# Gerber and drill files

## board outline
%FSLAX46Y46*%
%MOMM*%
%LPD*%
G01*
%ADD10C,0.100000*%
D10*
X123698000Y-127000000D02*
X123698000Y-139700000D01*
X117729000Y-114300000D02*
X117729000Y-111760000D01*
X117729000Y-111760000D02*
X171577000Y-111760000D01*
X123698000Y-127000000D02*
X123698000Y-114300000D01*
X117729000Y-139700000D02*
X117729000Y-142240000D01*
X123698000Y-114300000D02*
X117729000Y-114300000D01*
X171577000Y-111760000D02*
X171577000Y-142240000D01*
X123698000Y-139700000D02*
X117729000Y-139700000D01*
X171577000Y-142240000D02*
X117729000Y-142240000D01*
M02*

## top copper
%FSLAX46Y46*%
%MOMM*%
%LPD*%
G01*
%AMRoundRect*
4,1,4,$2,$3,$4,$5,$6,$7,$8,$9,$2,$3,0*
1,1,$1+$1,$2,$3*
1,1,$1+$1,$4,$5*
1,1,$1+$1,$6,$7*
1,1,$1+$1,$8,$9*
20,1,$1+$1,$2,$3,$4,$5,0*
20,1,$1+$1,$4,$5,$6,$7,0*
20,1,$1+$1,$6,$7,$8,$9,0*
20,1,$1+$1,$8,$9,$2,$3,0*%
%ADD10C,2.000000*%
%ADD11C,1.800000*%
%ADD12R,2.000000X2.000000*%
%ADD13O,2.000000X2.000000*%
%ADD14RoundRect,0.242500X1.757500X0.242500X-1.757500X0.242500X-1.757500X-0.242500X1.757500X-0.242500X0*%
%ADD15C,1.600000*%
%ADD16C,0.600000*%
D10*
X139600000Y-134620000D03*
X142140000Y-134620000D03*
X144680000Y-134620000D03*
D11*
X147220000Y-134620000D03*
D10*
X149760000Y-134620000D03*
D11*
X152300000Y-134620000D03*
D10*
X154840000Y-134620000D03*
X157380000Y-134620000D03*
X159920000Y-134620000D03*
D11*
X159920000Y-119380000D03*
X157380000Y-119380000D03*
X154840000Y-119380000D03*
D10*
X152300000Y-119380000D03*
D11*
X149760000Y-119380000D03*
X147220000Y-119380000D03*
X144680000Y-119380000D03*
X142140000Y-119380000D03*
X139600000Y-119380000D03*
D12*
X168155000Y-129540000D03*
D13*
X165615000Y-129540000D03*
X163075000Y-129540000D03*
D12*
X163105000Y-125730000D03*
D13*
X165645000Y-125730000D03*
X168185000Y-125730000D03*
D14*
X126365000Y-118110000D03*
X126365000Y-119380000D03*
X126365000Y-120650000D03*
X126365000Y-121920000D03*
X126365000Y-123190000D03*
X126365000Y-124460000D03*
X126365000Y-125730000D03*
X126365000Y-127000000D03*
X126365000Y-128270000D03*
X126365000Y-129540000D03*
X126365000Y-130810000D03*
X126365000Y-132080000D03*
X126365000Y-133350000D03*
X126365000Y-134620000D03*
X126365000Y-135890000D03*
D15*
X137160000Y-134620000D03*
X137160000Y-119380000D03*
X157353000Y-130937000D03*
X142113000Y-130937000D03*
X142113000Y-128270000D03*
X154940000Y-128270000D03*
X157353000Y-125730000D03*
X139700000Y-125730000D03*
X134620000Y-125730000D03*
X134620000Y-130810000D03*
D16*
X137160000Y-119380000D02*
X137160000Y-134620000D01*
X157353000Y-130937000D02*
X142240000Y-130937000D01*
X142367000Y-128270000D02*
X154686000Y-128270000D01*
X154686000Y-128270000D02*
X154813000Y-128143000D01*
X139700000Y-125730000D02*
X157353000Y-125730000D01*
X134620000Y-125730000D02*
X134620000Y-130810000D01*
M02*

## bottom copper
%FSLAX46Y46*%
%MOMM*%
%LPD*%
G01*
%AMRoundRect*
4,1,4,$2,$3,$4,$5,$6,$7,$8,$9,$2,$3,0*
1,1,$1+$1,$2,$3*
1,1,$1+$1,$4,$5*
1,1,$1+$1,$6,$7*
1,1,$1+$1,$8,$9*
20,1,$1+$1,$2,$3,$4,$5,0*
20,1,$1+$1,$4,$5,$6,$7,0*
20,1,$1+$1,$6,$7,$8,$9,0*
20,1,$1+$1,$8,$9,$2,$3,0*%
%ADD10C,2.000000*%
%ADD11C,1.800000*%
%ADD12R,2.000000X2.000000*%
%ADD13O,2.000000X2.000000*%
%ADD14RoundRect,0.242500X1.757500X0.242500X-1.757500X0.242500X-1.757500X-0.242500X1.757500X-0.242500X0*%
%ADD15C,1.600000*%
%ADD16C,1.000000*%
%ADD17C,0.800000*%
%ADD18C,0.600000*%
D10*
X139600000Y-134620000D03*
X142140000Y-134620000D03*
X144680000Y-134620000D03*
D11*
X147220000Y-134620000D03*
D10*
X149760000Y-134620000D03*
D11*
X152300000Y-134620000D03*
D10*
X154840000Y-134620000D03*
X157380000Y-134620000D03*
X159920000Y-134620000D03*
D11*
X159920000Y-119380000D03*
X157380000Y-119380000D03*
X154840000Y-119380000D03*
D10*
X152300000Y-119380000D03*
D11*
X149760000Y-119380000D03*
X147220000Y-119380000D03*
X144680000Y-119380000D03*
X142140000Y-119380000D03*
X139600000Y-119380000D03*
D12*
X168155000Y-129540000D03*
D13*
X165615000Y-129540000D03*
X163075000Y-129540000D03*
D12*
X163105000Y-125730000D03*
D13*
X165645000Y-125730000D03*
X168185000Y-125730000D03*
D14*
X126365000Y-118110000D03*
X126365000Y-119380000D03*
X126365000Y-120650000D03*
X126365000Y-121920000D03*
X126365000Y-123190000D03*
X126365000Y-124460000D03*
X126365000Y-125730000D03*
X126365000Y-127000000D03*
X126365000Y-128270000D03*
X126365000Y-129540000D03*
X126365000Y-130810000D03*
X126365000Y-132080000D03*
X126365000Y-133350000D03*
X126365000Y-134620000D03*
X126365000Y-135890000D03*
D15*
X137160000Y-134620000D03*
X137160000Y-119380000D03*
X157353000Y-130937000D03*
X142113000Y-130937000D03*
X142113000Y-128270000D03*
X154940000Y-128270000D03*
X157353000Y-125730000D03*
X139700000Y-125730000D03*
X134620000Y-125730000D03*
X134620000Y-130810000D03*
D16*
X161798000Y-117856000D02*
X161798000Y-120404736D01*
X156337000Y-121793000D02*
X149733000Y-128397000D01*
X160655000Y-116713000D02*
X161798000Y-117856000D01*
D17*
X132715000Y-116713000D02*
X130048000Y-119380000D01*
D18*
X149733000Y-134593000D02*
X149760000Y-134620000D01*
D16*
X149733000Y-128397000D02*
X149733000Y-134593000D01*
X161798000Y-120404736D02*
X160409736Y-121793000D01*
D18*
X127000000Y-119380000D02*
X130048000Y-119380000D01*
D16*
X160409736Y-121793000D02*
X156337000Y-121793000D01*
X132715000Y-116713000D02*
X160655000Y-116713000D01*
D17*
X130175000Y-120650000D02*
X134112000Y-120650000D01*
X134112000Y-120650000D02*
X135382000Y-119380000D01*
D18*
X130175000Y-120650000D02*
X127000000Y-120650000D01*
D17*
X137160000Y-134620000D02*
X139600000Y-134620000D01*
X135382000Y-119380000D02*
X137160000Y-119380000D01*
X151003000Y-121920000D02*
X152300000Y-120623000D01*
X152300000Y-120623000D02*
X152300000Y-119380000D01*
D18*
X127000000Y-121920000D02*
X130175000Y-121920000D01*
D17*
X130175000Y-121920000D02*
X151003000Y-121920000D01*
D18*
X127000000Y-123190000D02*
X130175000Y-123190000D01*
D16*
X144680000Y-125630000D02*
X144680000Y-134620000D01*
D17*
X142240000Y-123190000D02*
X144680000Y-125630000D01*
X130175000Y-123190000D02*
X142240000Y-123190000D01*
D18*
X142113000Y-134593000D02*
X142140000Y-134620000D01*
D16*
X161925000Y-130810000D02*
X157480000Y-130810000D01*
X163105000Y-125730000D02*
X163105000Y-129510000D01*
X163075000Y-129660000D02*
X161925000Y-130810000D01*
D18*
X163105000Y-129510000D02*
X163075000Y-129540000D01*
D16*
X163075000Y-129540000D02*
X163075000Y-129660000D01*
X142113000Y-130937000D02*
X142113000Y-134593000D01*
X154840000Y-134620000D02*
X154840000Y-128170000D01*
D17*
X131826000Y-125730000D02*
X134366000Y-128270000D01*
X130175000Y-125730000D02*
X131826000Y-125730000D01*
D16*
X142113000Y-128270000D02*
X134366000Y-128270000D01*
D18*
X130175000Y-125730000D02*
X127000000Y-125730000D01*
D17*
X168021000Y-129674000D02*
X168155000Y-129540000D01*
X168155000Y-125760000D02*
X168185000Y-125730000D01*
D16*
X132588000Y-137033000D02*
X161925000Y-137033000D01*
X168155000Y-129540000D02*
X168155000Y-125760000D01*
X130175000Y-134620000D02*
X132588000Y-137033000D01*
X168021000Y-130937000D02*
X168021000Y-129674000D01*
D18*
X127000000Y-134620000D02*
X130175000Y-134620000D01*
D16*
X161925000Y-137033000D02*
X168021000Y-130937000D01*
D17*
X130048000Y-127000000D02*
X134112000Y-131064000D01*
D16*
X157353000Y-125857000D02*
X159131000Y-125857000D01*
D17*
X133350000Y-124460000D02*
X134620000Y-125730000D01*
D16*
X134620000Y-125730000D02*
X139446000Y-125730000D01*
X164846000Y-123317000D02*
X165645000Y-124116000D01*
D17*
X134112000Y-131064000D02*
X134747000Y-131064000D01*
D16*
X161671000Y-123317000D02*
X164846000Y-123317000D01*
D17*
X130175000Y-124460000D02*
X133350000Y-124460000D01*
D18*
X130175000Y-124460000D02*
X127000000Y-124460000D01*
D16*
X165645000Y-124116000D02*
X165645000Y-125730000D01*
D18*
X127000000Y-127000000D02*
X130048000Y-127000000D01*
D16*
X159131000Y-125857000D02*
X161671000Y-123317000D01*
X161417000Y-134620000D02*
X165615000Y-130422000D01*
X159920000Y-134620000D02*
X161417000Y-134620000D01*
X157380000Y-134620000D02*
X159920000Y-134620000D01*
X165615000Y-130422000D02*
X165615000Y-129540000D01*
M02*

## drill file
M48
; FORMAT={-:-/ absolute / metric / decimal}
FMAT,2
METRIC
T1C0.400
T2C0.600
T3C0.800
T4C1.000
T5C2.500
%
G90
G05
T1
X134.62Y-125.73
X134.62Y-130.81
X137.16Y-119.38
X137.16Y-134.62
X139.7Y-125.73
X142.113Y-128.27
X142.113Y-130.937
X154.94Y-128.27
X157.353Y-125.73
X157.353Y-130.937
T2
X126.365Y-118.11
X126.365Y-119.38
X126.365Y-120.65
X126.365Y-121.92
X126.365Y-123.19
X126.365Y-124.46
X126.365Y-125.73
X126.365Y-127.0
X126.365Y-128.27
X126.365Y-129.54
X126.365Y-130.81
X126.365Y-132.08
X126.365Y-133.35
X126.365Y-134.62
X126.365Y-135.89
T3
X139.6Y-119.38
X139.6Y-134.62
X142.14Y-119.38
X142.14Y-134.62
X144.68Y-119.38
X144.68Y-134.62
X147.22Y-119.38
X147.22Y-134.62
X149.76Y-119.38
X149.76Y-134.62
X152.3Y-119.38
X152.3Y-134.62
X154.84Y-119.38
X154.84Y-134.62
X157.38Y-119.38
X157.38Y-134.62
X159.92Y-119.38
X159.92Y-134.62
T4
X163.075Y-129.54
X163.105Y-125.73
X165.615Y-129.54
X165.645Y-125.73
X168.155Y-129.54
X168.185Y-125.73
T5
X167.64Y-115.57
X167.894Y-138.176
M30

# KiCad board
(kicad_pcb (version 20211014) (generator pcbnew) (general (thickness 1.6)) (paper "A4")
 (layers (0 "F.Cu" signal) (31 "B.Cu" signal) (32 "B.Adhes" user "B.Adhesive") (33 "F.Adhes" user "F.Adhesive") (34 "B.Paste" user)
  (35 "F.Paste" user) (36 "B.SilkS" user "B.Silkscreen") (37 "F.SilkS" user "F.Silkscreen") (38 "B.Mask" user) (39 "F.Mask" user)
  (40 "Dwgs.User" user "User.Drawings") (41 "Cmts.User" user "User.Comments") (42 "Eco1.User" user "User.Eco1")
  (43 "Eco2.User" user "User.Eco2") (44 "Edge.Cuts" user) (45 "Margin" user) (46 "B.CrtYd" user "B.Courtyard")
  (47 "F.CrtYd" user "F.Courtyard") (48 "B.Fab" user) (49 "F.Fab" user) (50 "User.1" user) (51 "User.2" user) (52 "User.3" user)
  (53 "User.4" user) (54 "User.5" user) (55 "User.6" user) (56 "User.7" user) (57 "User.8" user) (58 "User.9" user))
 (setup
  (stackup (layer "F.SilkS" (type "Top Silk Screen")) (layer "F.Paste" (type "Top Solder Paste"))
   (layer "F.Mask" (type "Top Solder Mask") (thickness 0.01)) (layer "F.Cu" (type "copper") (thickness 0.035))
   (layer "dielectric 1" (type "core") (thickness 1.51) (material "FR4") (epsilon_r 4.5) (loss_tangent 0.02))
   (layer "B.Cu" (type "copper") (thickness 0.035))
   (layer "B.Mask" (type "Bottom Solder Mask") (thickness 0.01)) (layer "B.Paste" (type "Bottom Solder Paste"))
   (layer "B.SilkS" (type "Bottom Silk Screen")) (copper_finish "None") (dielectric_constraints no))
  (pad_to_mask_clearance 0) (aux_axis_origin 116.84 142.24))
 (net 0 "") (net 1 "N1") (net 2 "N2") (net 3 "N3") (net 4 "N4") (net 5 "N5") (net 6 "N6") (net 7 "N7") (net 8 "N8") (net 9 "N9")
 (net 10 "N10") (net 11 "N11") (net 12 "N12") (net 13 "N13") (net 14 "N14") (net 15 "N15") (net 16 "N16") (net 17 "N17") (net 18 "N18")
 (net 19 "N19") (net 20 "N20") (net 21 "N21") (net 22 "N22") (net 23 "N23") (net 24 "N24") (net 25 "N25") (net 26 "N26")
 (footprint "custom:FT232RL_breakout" (layer "F.Cu") (at 139.6 127 90)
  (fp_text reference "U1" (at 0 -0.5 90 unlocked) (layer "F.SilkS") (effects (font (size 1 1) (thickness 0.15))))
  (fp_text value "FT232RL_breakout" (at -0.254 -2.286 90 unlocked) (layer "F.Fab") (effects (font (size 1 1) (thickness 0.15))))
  (pad "1" thru_hole circle (at -7.62 0 90) (size 2 2) (drill 0.8) (layers *.Cu *.Mask) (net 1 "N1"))
  (pad "2" thru_hole circle (at -7.62 2.54 90) (size 2 2) (drill 0.8) (layers *.Cu *.Mask) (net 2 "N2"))
  (pad "3" thru_hole circle (at -7.62 5.08 90) (size 2 2) (drill 0.8) (layers *.Cu *.Mask) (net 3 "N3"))
  (pad "4" thru_hole circle (at -7.62 7.62 90) (size 1.8 1.8) (drill 0.8) (layers *.Cu *.Mask) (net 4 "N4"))
  (pad "5" thru_hole circle (at -7.62 10.16 90) (size 2 2) (drill 0.8) (layers *.Cu *.Mask) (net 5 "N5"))
  (pad "6" thru_hole circle (at -7.62 12.7 90) (size 1.8 1.8) (drill 0.8) (layers *.Cu *.Mask) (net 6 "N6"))
  (pad "7" thru_hole circle (at -7.62 15.24 90) (size 2 2) (drill 0.8) (layers *.Cu *.Mask) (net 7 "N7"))
  (pad "8" thru_hole circle (at -7.62 17.78 90) (size 2 2) (drill 0.8) (layers *.Cu *.Mask) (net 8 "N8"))
  (pad "9" thru_hole circle (at -7.62 20.32 90) (size 2 2) (drill 0.8) (layers *.Cu *.Mask) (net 8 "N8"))
  (pad "10" thru_hole circle (at 7.62 20.32 90) (size 1.8 1.8) (drill 0.8) (layers *.Cu *.Mask) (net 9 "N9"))
  (pad "11" thru_hole circle (at 7.62 17.78 90) (size 1.8 1.8) (drill 0.8) (layers *.Cu *.Mask) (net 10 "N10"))
  (pad "12" thru_hole circle (at 7.62 15.24 90) (size 1.8 1.8) (drill 0.8) (layers *.Cu *.Mask) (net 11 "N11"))
  (pad "13" thru_hole circle (at 7.62 12.7 90) (size 2 2) (drill 0.8) (layers *.Cu *.Mask) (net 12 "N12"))
  (pad "14" thru_hole circle (at 7.62 10.16 90) (size 1.8 1.8) (drill 0.8) (layers *.Cu *.Mask) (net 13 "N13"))
  (pad "15" thru_hole circle (at 7.62 7.62 90) (size 1.8 1.8) (drill 0.8) (layers *.Cu *.Mask) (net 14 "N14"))
  (pad "16" thru_hole circle (at 7.62 5.08 90) (size 1.8 1.8) (drill 0.8) (layers *.Cu *.Mask) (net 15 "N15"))
  (pad "17" thru_hole circle (at 7.62 2.54 90) (size 1.8 1.8) (drill 0.8) (layers *.Cu *.Mask) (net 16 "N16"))
  (pad "18" thru_hole circle (at 7.62 0 90) (size 1.8 1.8) (drill 0.8) (layers *.Cu *.Mask) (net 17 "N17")))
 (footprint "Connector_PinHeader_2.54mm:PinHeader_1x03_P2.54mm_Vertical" (layer "F.Cu") (at 168.155 129.54 -90)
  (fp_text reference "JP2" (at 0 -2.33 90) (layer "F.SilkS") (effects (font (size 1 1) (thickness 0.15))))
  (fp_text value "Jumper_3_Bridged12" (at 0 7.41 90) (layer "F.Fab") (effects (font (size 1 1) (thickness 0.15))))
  (pad "1" thru_hole rect locked (at 0 0 270) (size 2 2) (drill 1) (layers *.Cu *.Mask) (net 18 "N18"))
  (pad "2" thru_hole oval locked (at 0 2.54 270) (size 2 2) (drill 1) (layers *.Cu *.Mask) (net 8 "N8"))
  (pad "3" thru_hole oval locked (at 0 5.08 270) (size 2 2) (drill 1) (layers *.Cu *.Mask) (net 2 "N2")))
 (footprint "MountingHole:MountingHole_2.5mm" (layer "F.Cu") (at 167.894 138.176)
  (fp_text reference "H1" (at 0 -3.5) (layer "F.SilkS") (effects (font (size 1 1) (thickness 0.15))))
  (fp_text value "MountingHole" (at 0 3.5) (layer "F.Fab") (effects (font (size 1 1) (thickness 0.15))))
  (pad "" np_thru_hole circle locked (at 0 0) (size 2.5 2.5) (drill 2.5) (layers *.Cu *.Mask)))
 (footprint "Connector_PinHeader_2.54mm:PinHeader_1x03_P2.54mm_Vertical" (layer "F.Cu") (at 163.105 125.73 90)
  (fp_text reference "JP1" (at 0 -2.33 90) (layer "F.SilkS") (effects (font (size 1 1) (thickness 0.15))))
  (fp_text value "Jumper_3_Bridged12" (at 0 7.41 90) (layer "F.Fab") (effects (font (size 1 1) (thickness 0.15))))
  (pad "1" thru_hole rect locked (at 0 0 90) (size 2 2) (drill 1) (layers *.Cu *.Mask) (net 2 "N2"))
  (pad "2" thru_hole oval locked (at 0 2.54 90) (size 2 2) (drill 1) (layers *.Cu *.Mask) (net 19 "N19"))
  (pad "3" thru_hole oval locked (at 0 5.08 90) (size 2 2) (drill 1) (layers *.Cu *.Mask) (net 18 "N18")))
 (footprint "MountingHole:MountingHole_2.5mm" (layer "F.Cu") (at 167.64 115.57)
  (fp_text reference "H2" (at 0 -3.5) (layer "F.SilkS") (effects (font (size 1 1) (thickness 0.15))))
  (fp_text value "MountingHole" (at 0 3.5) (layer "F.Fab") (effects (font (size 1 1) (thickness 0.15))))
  (pad "" np_thru_hole circle locked (at 0 0) (size 2.5 2.5) (drill 2.5) (layers *.Cu *.Mask)))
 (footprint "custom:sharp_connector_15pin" (layer "B.Cu") (at 126.365 127 180)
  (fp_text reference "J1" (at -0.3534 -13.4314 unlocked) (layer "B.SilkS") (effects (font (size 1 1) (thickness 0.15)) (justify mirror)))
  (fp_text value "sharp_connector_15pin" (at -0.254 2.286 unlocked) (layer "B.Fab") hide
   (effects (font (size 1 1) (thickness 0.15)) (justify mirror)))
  (pad "1" thru_hole roundrect (at 0 8.89 180) (size 4 0.97) (drill 0.6) (layers *.Cu *.Mask) (roundrect_rratio 0.25) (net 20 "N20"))
  (pad "2" thru_hole roundrect (at 0 7.62 180) (size 4 0.97) (drill 0.6) (layers *.Cu *.Mask) (roundrect_rratio 0.25) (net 5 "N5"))
  (pad "3" thru_hole roundrect (at 0 6.35 180) (size 4 0.97) (drill 0.6) (layers *.Cu *.Mask) (roundrect_rratio 0.25) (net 1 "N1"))
  (pad "4" thru_hole roundrect (at 0 5.08 180) (size 4 0.97) (drill 0.6) (layers *.Cu *.Mask) (roundrect_rratio 0.25) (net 12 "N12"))
  (pad "5" thru_hole roundrect (at 0 3.81 180) (size 4 0.97) (drill 0.6) (layers *.Cu *.Mask) (roundrect_rratio 0.25) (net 3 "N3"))
  (pad "6" thru_hole roundrect (at 0 2.54 180) (size 4 0.97) (drill 0.6) (layers *.Cu *.Mask) (roundrect_rratio 0.25) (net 19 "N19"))
  (pad "7" thru_hole roundrect (at 0 1.27 180) (size 4 0.97) (drill 0.6) (layers *.Cu *.Mask) (roundrect_rratio 0.25) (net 7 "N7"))
  (pad "8" thru_hole roundrect (at 0 0 180) (size 4 0.97) (drill 0.6) (layers *.Cu *.Mask) (roundrect_rratio 0.25) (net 19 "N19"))
  (pad "9" thru_hole roundrect (at 0 -1.27 180) (size 4 0.97) (drill 0.6) (layers *.Cu *.Mask) (roundrect_rratio 0.25) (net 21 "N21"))
  (pad "10" thru_hole roundrect (at 0 -2.54 180) (size 4 0.97) (drill 0.6) (layers *.Cu *.Mask) (roundrect_rratio 0.25) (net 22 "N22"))
  (pad "11" thru_hole roundrect (at 0 -3.81 180) (size 4 0.97) (drill 0.6) (layers *.Cu *.Mask) (roundrect_rratio 0.25) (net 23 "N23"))
  (pad "12" thru_hole roundrect (at 0 -5.08 180) (size 4 0.97) (drill 0.6) (layers *.Cu *.Mask) (roundrect_rratio 0.25) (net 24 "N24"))
  (pad "13" thru_hole roundrect (at 0 -6.35 180) (size 4 0.97) (drill 0.6) (layers *.Cu *.Mask) (roundrect_rratio 0.25) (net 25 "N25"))
  (pad "14" thru_hole roundrect (at 0 -7.62 180) (size 4 0.97) (drill 0.6) (layers *.Cu *.Mask) (roundrect_rratio 0.25) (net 18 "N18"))
  (pad "15" thru_hole roundrect (at 0 -8.89 180) (size 4 0.97) (drill 0.6) (layers *.Cu *.Mask) (roundrect_rratio 0.25) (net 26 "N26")))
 (gr_line (start 123.698 127) (end 123.698 139.7) (layer "Edge.Cuts") (width 0.1))
 (gr_line (start 117.729 114.3) (end 117.729 111.76) (layer "Edge.Cuts") (width 0.1))
 (gr_line (start 117.729 111.76) (end 171.577 111.76) (layer "Edge.Cuts") (width 0.1))
 (gr_line (start 123.698 127) (end 123.698 114.3) (layer "Edge.Cuts") (width 0.1))
 (gr_line (start 117.729 139.7) (end 117.729 142.24) (layer "Edge.Cuts") (width 0.1))
 (gr_line (start 123.698 114.3) (end 117.729 114.3) (layer "Edge.Cuts") (width 0.1))
 (gr_line (start 171.577 111.76) (end 171.577 142.24) (layer "Edge.Cuts") (width 0.1))
 (gr_line (start 123.698 139.7) (end 117.729 139.7) (layer "Edge.Cuts") (width 0.1))
 (gr_line (start 171.577 142.24) (end 117.729 142.24) (layer "Edge.Cuts") (width 0.1))
 (segment (start 161.798 117.856) (end 161.798 120.404736) (width 1) (layer "B.Cu") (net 5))
 (segment (start 156.337 121.793) (end 149.733 128.397) (width 1) (layer "B.Cu") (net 5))
 (segment (start 160.655 116.713) (end 161.798 117.856) (width 1) (layer "B.Cu") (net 5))
 (segment (start 132.715 116.713) (end 130.048 119.38) (width 0.8) (layer "B.Cu") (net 5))
 (segment (start 149.733 134.593) (end 149.76 134.62) (width 0.6) (layer "B.Cu") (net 5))
 (segment (start 149.733 128.397) (end 149.733 134.593) (width 1) (layer "B.Cu") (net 5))
 (segment (start 161.798 120.404736) (end 160.409736 121.793) (width 1) (layer "B.Cu") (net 5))
 (segment (start 127 119.38) (end 130.048 119.38) (width 0.6) (layer "B.Cu") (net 5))
 (segment (start 160.409736 121.793) (end 156.337 121.793) (width 1) (layer "B.Cu") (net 5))
 (segment (start 132.715 116.713) (end 160.655 116.713) (width 1) (layer "B.Cu") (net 5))
 (segment (start 137.16 119.38) (end 137.16 134.62) (width 0.6) (layer "F.Cu") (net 1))
 (via (at 137.16 134.62) (size 1.6) (drill 0.4) (layers "F.Cu" "B.Cu") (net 1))
 (via (at 137.16 119.38) (size 1.6) (drill 0.4) (layers "F.Cu" "B.Cu") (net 1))
 (segment (start 130.175 120.65) (end 134.112 120.65) (width 0.8) (layer "B.Cu") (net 1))
 (segment (start 134.112 120.65) (end 135.382 119.38) (width 0.8) (layer "B.Cu") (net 1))
 (segment (start 130.175 120.65) (end 127 120.65) (width 0.6) (layer "B.Cu") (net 1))
 (segment (start 137.16 134.62) (end 139.6 134.62) (width 0.8) (layer "B.Cu") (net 1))
 (segment (start 135.382 119.38) (end 137.16 119.38) (width 0.8) (layer "B.Cu") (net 1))
 (segment (start 151.003 121.92) (end 152.3 120.623) (width 0.8) (layer "B.Cu") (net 12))
 (segment (start 152.3 120.623) (end 152.3 119.38) (width 0.8) (layer "B.Cu") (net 12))
 (segment (start 127 121.92) (end 130.175 121.92) (width 0.6) (layer "B.Cu") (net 12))
 (segment (start 130.175 121.92) (end 151.003 121.92) (width 0.8) (layer "B.Cu") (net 12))
 (segment (start 127 123.19) (end 130.175 123.19) (width 0.6) (layer "B.Cu") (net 3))
 (segment (start 144.68 125.63) (end 144.68 134.62) (width 1) (layer "B.Cu") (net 3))
 (segment (start 142.24 123.19) (end 144.68 125.63) (width 0.8) (layer "B.Cu") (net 3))
 (segment (start 130.175 123.19) (end 142.24 123.19) (width 0.8) (layer "B.Cu") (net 3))
 (segment (start 157.353 130.937) (end 142.24 130.937) (width 0.6) (layer "F.Cu") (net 2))
 (via (at 157.353 130.937) (size 1.6) (drill 0.4) (layers "F.Cu" "B.Cu") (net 2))
 (via (at 142.113 130.937) (size 1.6) (drill 0.4) (layers "F.Cu" "B.Cu") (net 2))
 (segment (start 142.113 134.593) (end 142.14 134.62) (width 0.6) (layer "B.Cu") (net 2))
 (segment (start 161.925 130.81) (end 157.48 130.81) (width 1) (layer "B.Cu") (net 2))
 (segment (start 163.105 125.73) (end 163.105 129.51) (width 1) (layer "B.Cu") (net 2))
 (segment (start 163.075 129.66) (end 161.925 130.81) (width 1) (layer "B.Cu") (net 2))
 (segment (start 163.105 129.51) (end 163.075 129.54) (width 0.6) (layer "B.Cu") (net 2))
 (segment (start 163.075 129.54) (end 163.075 129.66) (width 1) (layer "B.Cu") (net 2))
 (segment (start 142.113 130.937) (end 142.113 134.593) (width 1) (layer "B.Cu") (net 2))
 (segment (start 142.367 128.27) (end 154.686 128.27) (width 0.6) (layer "F.Cu") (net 7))
 (segment (start 154.686 128.27) (end 154.813 128.143) (width 0.6) (layer "F.Cu") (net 7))
 (via (at 142.113 128.27) (size 1.6) (drill 0.4) (layers "F.Cu" "B.Cu") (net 7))
 (via (at 154.94 128.27) (size 1.6) (drill 0.4) (layers "F.Cu" "B.Cu") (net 7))
 (segment (start 154.84 134.62) (end 154.84 128.17) (width 1) (layer "B.Cu") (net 7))
 (segment (start 131.826 125.73) (end 134.366 128.27) (width 0.8) (layer "B.Cu") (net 7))
 (segment (start 130.175 125.73) (end 131.826 125.73) (width 0.8) (layer "B.Cu") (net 7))
 (segment (start 142.113 128.27) (end 134.366 128.27) (width 1) (layer "B.Cu") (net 7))
 (segment (start 130.175 125.73) (end 127 125.73) (width 0.6) (layer "B.Cu") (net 7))
 (segment (start 168.021 129.674) (end 168.155 129.54) (width 0.8) (layer "B.Cu") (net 18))
 (segment (start 168.155 125.76) (end 168.185 125.73) (width 0.8) (layer "B.Cu") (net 18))
 (segment (start 132.588 137.033) (end 161.925 137.033) (width 1) (layer "B.Cu") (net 18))
 (segment (start 168.155 129.54) (end 168.155 125.76) (width 1) (layer "B.Cu") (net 18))
 (segment (start 130.175 134.62) (end 132.588 137.033) (width 1) (layer "B.Cu") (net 18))
 (segment (start 168.021 130.937) (end 168.021 129.674) (width 1) (layer "B.Cu") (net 18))
 (segment (start 127 134.62) (end 130.175 134.62) (width 0.6) (layer "B.Cu") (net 18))
 (segment (start 161.925 137.033) (end 168.021 130.937) (width 1) (layer "B.Cu") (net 18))
 (segment (start 139.7 125.73) (end 157.353 125.73) (width 0.6) (layer "F.Cu") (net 19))
 (segment (start 134.62 125.73) (end 134.62 130.81) (width 0.6) (layer "F.Cu") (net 19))
 (via (at 157.353 125.73) (size 1.6) (drill 0.4) (layers "F.Cu" "B.Cu") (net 19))
 (via (at 139.7 125.73) (size 1.6) (drill 0.4) (layers "F.Cu" "B.Cu") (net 19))
 (via (at 134.62 125.73) (size 1.6) (drill 0.4) (layers "F.Cu" "B.Cu") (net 19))
 (via (at 134.62 130.81) (size 1.6) (drill 0.4) (layers "F.Cu" "B.Cu") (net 19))
 (segment (start 130.048 127) (end 134.112 131.064) (width 0.8) (layer "B.Cu") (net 19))
 (segment (start 157.353 125.857) (end 159.131 125.857) (width 1) (layer "B.Cu") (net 19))
 (segment (start 133.35 124.46) (end 134.62 125.73) (width 0.8) (layer "B.Cu") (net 19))
 (segment (start 134.62 125.73) (end 139.446 125.73) (width 1) (layer "B.Cu") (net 19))
 (segment (start 164.846 123.317) (end 165.645 124.116) (width 1) (layer "B.Cu") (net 19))
 (segment (start 134.112 131.064) (end 134.747 131.064) (width 0.8) (layer "B.Cu") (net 19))
 (segment (start 161.671 123.317) (end 164.846 123.317) (width 1) (layer "B.Cu") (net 19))
 (segment (start 130.175 124.46) (end 133.35 124.46) (width 0.8) (layer "B.Cu") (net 19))
 (segment (start 130.175 124.46) (end 127 124.46) (width 0.6) (layer "B.Cu") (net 19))
 (segment (start 165.645 124.116) (end 165.645 125.73) (width 1) (layer "B.Cu") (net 19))
 (segment (start 127 127) (end 130.048 127) (width 0.6) (layer "B.Cu") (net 19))
 (segment (start 159.131 125.857) (end 161.671 123.317) (width 1) (layer "B.Cu") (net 19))
 (segment (start 161.417 134.62) (end 165.615 130.422) (width 1) (layer "B.Cu") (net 8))
 (segment (start 159.92 134.62) (end 161.417 134.62) (width 1) (layer "B.Cu") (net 8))
 (segment (start 157.38 134.62) (end 159.92 134.62) (width 1) (layer "B.Cu") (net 8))
 (segment (start 165.615 130.422) (end 165.615 129.54) (width 1) (layer "B.Cu") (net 8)))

